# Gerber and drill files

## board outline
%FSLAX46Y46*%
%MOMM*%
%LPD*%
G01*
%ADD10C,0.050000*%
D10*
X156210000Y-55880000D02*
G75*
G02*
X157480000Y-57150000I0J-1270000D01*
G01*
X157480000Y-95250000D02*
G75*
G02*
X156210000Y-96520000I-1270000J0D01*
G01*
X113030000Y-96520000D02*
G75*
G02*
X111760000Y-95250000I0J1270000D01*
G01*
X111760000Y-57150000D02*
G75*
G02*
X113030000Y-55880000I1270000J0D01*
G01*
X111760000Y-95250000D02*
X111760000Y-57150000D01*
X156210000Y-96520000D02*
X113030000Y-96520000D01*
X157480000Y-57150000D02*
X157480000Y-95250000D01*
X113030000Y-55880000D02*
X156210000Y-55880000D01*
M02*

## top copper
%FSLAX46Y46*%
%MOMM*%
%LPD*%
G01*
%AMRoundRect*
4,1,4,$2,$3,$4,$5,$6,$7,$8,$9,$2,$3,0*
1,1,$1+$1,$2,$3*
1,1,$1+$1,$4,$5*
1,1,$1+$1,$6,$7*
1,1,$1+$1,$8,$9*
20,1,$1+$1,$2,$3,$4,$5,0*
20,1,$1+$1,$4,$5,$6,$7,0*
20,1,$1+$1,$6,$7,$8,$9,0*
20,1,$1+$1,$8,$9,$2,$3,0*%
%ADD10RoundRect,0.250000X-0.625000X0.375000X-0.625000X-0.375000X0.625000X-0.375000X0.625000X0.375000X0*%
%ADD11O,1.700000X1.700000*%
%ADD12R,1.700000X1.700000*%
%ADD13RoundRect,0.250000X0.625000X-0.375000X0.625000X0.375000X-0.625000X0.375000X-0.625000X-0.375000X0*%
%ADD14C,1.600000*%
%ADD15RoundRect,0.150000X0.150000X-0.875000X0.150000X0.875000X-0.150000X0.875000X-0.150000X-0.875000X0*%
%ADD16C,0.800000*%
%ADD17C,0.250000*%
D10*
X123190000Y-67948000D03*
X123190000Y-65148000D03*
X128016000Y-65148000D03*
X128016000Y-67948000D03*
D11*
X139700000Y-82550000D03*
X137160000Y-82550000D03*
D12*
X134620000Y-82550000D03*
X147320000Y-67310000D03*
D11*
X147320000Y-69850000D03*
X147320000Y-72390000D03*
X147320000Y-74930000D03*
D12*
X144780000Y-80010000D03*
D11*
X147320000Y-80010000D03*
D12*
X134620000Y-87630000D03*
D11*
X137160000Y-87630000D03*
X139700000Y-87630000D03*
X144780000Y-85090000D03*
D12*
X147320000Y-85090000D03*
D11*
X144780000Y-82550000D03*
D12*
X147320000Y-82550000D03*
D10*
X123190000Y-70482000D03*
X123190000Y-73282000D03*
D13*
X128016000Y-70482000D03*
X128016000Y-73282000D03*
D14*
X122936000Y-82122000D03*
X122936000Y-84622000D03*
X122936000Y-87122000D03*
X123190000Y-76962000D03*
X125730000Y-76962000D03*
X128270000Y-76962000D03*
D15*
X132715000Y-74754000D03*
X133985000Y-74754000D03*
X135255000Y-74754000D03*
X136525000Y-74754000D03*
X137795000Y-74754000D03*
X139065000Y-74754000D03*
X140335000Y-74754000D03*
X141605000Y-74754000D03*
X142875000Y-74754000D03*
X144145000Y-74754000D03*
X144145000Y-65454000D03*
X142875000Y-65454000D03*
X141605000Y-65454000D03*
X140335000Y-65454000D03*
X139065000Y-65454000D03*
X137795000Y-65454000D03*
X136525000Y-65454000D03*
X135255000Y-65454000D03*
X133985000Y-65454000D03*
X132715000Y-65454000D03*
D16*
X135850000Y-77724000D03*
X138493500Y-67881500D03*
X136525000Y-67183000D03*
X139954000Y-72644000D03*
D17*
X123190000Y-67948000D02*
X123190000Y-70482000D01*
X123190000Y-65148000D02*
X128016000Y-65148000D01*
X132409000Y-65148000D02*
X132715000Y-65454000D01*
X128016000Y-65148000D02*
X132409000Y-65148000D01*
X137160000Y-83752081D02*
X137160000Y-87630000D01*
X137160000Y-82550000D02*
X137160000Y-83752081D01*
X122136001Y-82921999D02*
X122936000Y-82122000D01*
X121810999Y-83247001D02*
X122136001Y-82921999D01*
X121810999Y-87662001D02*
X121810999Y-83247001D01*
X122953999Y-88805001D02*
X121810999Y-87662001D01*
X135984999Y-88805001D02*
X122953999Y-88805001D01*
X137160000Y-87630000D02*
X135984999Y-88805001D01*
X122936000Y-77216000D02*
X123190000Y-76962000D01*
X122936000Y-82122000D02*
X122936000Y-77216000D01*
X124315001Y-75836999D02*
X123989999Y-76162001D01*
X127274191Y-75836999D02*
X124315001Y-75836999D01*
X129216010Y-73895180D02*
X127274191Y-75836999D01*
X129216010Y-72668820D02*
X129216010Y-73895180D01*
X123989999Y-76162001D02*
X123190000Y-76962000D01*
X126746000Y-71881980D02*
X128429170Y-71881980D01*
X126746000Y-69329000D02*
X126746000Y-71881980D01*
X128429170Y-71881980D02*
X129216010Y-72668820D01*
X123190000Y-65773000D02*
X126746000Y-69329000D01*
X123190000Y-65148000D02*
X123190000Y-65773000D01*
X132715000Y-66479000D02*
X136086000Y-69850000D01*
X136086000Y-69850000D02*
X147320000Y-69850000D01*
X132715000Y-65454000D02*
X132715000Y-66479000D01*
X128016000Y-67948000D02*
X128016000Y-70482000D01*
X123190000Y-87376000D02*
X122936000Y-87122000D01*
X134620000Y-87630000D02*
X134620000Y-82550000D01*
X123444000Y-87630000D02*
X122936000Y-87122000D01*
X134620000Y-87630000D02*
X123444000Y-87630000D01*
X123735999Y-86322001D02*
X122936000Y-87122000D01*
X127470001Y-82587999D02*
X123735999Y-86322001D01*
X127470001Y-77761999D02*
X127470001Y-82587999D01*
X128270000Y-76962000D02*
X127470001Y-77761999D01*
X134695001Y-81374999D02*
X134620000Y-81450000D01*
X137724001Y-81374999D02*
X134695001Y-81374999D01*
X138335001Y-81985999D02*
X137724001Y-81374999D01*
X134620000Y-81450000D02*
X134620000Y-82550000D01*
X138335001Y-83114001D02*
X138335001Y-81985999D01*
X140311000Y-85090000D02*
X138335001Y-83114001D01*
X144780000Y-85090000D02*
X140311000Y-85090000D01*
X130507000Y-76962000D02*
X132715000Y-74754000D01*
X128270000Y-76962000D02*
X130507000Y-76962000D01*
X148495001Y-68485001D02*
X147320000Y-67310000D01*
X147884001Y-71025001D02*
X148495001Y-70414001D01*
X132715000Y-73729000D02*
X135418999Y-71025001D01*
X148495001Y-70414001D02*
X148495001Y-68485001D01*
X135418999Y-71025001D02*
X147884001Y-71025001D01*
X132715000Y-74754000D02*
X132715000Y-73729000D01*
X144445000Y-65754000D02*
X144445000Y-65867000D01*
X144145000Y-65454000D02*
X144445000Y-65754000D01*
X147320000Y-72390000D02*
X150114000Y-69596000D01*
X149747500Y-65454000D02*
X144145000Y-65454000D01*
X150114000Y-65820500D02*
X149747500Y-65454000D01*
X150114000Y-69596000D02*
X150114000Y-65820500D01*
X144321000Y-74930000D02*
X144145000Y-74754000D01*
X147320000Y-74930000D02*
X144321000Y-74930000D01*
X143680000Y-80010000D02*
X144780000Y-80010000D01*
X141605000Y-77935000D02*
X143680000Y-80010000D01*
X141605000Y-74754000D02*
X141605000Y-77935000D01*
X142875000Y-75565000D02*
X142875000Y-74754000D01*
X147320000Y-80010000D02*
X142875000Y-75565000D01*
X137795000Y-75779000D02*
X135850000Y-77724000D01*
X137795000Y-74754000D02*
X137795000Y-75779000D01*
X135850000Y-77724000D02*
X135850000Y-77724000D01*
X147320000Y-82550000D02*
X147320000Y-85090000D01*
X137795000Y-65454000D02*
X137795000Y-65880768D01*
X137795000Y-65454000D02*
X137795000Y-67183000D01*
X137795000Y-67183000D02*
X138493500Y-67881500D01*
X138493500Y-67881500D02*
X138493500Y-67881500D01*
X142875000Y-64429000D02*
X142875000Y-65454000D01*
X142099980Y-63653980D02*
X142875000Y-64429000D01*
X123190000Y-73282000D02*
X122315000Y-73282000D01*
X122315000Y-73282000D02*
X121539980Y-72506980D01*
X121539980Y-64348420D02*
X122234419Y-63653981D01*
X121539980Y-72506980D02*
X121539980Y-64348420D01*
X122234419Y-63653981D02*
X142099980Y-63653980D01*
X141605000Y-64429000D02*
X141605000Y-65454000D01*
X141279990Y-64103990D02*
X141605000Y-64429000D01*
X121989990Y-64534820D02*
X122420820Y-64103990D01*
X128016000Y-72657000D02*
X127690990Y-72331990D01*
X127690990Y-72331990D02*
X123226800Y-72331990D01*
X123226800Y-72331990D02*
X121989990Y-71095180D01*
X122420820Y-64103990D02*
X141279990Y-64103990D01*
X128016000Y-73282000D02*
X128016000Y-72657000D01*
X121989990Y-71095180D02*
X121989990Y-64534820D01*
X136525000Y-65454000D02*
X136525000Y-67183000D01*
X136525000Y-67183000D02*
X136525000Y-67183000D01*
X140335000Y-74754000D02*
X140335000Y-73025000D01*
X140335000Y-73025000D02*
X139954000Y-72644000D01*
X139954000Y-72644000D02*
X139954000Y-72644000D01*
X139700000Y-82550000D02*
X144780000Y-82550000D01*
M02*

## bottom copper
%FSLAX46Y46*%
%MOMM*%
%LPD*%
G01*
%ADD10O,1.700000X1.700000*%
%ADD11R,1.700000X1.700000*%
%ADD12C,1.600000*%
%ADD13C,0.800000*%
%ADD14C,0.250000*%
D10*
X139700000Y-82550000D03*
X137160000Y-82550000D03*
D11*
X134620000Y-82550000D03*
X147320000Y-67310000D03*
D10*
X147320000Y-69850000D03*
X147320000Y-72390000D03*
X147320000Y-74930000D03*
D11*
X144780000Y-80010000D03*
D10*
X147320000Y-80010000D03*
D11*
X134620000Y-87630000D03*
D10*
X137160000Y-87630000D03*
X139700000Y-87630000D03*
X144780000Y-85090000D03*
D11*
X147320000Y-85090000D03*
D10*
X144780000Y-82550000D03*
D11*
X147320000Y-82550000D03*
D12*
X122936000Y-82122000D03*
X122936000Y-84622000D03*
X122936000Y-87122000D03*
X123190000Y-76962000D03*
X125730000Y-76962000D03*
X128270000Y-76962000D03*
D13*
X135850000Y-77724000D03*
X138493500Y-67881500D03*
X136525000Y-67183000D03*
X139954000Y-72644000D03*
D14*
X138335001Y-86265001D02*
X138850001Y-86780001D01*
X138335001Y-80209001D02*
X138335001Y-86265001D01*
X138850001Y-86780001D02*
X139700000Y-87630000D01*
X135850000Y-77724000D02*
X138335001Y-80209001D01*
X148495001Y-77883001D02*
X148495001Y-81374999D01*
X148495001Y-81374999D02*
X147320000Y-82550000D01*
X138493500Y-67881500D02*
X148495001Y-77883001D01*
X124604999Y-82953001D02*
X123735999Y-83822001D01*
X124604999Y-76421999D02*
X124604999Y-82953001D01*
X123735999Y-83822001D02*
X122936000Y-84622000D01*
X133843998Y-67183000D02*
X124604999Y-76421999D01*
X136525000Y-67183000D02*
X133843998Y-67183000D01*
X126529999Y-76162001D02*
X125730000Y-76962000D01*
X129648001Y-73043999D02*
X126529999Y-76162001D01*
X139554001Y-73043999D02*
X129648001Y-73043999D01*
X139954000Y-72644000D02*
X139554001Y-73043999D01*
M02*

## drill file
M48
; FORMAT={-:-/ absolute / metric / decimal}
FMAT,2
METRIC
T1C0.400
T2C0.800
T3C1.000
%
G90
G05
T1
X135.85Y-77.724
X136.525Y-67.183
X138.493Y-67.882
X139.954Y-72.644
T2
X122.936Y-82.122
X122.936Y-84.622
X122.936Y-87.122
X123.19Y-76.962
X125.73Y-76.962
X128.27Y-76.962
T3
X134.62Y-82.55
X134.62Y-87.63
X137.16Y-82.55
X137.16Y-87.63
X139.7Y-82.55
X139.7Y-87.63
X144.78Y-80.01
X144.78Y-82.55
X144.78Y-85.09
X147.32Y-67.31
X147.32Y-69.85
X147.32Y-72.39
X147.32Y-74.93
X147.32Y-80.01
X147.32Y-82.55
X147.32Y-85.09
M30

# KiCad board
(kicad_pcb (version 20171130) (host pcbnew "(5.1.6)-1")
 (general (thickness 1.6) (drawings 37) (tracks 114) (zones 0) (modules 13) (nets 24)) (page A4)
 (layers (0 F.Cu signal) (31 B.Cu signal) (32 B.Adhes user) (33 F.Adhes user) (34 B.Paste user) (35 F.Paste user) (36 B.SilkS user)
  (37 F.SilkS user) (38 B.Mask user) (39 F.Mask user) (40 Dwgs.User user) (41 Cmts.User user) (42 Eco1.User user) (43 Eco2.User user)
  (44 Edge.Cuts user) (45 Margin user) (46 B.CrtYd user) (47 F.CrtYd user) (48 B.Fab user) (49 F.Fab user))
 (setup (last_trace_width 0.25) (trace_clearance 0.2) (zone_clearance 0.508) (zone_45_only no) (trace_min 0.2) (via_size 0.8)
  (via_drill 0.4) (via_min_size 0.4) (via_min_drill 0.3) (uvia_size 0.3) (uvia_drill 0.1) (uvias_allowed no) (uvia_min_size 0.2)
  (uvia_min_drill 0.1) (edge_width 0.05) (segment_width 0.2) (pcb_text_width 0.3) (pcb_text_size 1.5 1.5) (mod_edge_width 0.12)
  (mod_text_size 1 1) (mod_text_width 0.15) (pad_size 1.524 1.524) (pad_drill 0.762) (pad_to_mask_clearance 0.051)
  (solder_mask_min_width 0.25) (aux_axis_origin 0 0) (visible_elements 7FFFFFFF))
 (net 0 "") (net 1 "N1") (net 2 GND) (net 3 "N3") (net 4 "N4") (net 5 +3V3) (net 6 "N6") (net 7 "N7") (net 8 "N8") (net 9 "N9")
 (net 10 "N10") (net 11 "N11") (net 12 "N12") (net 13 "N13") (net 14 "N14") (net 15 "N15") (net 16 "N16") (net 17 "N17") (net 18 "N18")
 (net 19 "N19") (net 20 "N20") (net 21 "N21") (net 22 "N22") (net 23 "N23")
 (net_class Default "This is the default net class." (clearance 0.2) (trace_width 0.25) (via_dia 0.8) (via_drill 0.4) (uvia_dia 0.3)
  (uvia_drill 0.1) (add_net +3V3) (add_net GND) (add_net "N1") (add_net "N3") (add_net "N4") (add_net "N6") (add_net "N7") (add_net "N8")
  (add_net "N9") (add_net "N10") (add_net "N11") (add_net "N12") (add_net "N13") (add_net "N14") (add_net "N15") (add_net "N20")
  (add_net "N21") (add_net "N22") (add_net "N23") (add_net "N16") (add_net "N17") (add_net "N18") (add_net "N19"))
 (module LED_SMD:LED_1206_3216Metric (layer F.Cu) (at 123.19 66.548 270)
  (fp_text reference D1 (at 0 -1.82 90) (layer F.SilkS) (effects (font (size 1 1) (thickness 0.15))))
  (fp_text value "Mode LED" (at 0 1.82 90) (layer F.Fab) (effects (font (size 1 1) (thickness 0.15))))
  (pad 2 smd roundrect (at 1.4 0 270) (size 1.25 1.75) (layers F.Cu F.Paste F.Mask) (roundrect_rratio 0.2) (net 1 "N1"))
  (pad 1 smd roundrect (at -1.4 0 270) (size 1.25 1.75) (layers F.Cu F.Paste F.Mask) (roundrect_rratio 0.2) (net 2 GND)))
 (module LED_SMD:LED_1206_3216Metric (layer F.Cu) (at 128.016 66.548 270)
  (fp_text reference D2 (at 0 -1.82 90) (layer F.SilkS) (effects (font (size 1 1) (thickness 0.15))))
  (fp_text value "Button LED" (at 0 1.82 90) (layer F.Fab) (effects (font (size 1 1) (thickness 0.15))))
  (pad 1 smd roundrect (at -1.4 0 270) (size 1.25 1.75) (layers F.Cu F.Paste F.Mask) (roundrect_rratio 0.2) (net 2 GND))
  (pad 2 smd roundrect (at 1.4 0 270) (size 1.25 1.75) (layers F.Cu F.Paste F.Mask) (roundrect_rratio 0.2) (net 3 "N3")))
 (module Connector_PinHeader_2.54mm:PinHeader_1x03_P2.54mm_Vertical (layer F.Cu) (at 134.62 82.55 90)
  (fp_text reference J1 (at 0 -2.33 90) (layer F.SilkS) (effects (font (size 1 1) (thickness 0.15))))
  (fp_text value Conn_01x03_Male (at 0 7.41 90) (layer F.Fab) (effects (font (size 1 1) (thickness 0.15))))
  (pad 3 thru_hole oval (at 0 5.08 90) (size 1.7 1.7) (drill 1) (layers *.Cu *.Mask) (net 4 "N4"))
  (pad 2 thru_hole oval (at 0 2.54 90) (size 1.7 1.7) (drill 1) (layers *.Cu *.Mask) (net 2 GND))
  (pad 1 thru_hole rect (at 0 0 90) (size 1.7 1.7) (drill 1) (layers *.Cu *.Mask) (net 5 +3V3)))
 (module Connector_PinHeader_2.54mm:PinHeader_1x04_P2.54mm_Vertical (layer F.Cu) (at 147.32 67.31)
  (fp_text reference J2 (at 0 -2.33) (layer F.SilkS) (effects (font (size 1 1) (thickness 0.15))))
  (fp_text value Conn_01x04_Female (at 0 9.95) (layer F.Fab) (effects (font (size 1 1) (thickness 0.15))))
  (pad 1 thru_hole rect (at 0 0) (size 1.7 1.7) (drill 1) (layers *.Cu *.Mask) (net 5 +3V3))
  (pad 2 thru_hole oval (at 0 2.54) (size 1.7 1.7) (drill 1) (layers *.Cu *.Mask) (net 2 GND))
  (pad 3 thru_hole oval (at 0 5.08) (size 1.7 1.7) (drill 1) (layers *.Cu *.Mask) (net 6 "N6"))
  (pad 4 thru_hole oval (at 0 7.62) (size 1.7 1.7) (drill 1) (layers *.Cu *.Mask) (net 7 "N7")))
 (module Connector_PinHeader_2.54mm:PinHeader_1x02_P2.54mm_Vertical (layer F.Cu) (at 144.78 80.01 90)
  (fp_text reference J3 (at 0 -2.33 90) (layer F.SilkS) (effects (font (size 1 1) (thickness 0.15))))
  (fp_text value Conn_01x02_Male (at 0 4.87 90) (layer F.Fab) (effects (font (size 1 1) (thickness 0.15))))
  (pad 1 thru_hole rect (at 0 0 90) (size 1.7 1.7) (drill 1) (layers *.Cu *.Mask) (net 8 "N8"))
  (pad 2 thru_hole oval (at 0 2.54 90) (size 1.7 1.7) (drill 1) (layers *.Cu *.Mask) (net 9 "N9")))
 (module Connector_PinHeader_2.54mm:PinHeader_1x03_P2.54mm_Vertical (layer F.Cu) (at 134.62 87.63 90)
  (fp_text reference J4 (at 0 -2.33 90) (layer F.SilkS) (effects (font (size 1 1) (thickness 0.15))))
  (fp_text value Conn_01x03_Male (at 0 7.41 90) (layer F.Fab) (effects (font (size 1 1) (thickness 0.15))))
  (pad 1 thru_hole rect (at 0 0 90) (size 1.7 1.7) (drill 1) (layers *.Cu *.Mask) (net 5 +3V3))
  (pad 2 thru_hole oval (at 0 2.54 90) (size 1.7 1.7) (drill 1) (layers *.Cu *.Mask) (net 2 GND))
  (pad 3 thru_hole oval (at 0 5.08 90) (size 1.7 1.7) (drill 1) (layers *.Cu *.Mask) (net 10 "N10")))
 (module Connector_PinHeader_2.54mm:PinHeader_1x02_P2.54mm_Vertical (layer F.Cu) (at 147.32 85.09 270)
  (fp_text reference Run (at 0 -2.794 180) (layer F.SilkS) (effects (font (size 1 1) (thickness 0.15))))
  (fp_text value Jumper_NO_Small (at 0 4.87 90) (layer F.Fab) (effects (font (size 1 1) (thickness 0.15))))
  (pad 2 thru_hole oval (at 0 2.54 270) (size 1.7 1.7) (drill 1) (layers *.Cu *.Mask) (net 5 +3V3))
  (pad 1 thru_hole rect (at 0 0 270) (size 1.7 1.7) (drill 1) (layers *.Cu *.Mask) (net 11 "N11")))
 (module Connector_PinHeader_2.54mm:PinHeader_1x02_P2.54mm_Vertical (layer F.Cu) (at 147.32 82.55 270)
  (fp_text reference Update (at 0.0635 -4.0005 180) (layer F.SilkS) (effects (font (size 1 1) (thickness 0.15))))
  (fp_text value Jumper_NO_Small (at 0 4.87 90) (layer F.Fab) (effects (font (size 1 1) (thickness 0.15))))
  (pad 2 thru_hole oval (at 0 2.54 270) (size 1.7 1.7) (drill 1) (layers *.Cu *.Mask) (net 4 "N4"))
  (pad 1 thru_hole rect (at 0 0 270) (size 1.7 1.7) (drill 1) (layers *.Cu *.Mask) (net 11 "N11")))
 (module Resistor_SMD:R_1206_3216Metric (layer F.Cu) (at 123.19 71.882 270)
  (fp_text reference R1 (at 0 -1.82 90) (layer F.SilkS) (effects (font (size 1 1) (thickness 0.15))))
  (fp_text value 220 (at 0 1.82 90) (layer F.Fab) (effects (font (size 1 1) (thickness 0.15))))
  (pad 1 smd roundrect (at -1.4 0 270) (size 1.25 1.75) (layers F.Cu F.Paste F.Mask) (roundrect_rratio 0.2) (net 1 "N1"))
  (pad 2 smd roundrect (at 1.4 0 270) (size 1.25 1.75) (layers F.Cu F.Paste F.Mask) (roundrect_rratio 0.2) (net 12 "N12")))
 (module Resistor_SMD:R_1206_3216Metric (layer F.Cu) (at 128.016 71.882 90)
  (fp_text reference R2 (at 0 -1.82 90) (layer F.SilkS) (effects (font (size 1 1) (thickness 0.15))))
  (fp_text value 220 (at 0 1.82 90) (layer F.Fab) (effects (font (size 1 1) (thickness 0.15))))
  (pad 2 smd roundrect (at 1.4 0 90) (size 1.25 1.75) (layers F.Cu F.Paste F.Mask) (roundrect_rratio 0.2) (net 3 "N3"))
  (pad 1 smd roundrect (at -1.4 0 90) (size 1.25 1.75) (layers F.Cu F.Paste F.Mask) (roundrect_rratio 0.2) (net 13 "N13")))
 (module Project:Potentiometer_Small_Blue (layer F.Cu) (at 122.936 87.122)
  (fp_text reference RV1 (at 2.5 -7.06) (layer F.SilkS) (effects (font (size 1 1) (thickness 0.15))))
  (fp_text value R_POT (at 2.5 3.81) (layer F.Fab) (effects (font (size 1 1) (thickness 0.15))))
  (pad 3 thru_hole circle (at 0 -5) (size 1.6 1.6) (drill 0.8) (layers *.Cu *.Mask) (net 2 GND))
  (pad 2 thru_hole circle (at 0 -2.5) (size 1.6 1.6) (drill 0.8) (layers *.Cu *.Mask) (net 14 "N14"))
  (pad 1 thru_hole circle (at 0 0) (size 1.6 1.6) (drill 0.8) (layers *.Cu *.Mask) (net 5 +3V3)))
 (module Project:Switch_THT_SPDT (layer F.Cu) (at 125.73 76.962)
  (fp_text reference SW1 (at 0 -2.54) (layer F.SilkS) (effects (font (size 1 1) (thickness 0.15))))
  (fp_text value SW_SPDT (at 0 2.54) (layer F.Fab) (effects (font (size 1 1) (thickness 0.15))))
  (pad 1 thru_hole circle (at -2.54 0) (size 1.6 1.6) (drill 0.8) (layers *.Cu *.Mask) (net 2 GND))
  (pad 2 thru_hole circle (at 0 0) (size 1.6 1.6) (drill 0.8) (layers *.Cu *.Mask) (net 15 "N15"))
  (pad 3 thru_hole circle (at 2.54 0) (size 1.6 1.6) (drill 0.8) (layers *.Cu *.Mask) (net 5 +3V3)))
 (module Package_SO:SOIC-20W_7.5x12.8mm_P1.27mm (layer F.Cu) (at 138.43 70.104 90)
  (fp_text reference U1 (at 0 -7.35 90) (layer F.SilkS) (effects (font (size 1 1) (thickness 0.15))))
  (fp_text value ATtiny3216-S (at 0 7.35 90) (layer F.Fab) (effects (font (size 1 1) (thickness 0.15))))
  (pad 1 smd roundrect (at -4.65 -5.715 90) (size 2.05 0.6) (layers F.Cu F.Paste F.Mask) (roundrect_rratio 0.25) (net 5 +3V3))
  (pad 2 smd roundrect (at -4.65 -4.445 90) (size 2.05 0.6) (layers F.Cu F.Paste F.Mask) (roundrect_rratio 0.25) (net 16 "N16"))
  (pad 3 smd roundrect (at -4.65 -3.175 90) (size 2.05 0.6) (layers F.Cu F.Paste F.Mask) (roundrect_rratio 0.25) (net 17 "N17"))
  (pad 4 smd roundrect (at -4.65 -1.905 90) (size 2.05 0.6) (layers F.Cu F.Paste F.Mask) (roundrect_rratio 0.25) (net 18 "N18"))
  (pad 5 smd roundrect (at -4.65 -0.635 90) (size 2.05 0.6) (layers F.Cu F.Paste F.Mask) (roundrect_rratio 0.25) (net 10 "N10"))
  (pad 6 smd roundrect (at -4.65 0.635 90) (size 2.05 0.6) (layers F.Cu F.Paste F.Mask) (roundrect_rratio 0.25) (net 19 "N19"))
  (pad 7 smd roundrect (at -4.65 1.905 90) (size 2.05 0.6) (layers F.Cu F.Paste F.Mask) (roundrect_rratio 0.25) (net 15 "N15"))
  (pad 8 smd roundrect (at -4.65 3.175 90) (size 2.05 0.6) (layers F.Cu F.Paste F.Mask) (roundrect_rratio 0.25) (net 8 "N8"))
  (pad 9 smd roundrect (at -4.65 4.445 90) (size 2.05 0.6) (layers F.Cu F.Paste F.Mask) (roundrect_rratio 0.25) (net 9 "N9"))
  (pad 10 smd roundrect (at -4.65 5.715 90) (size 2.05 0.6) (layers F.Cu F.Paste F.Mask) (roundrect_rratio 0.25) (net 7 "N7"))
  (pad 11 smd roundrect (at 4.65 5.715 90) (size 2.05 0.6) (layers F.Cu F.Paste F.Mask) (roundrect_rratio 0.25) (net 6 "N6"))
  (pad 12 smd roundrect (at 4.65 4.445 90) (size 2.05 0.6) (layers F.Cu F.Paste F.Mask) (roundrect_rratio 0.25) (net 12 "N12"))
  (pad 13 smd roundrect (at 4.65 3.175 90) (size 2.05 0.6) (layers F.Cu F.Paste F.Mask) (roundrect_rratio 0.25) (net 13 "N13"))
  (pad 14 smd roundrect (at 4.65 1.905 90) (size 2.05 0.6) (layers F.Cu F.Paste F.Mask) (roundrect_rratio 0.25) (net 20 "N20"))
  (pad 15 smd roundrect (at 4.65 0.635 90) (size 2.05 0.6) (layers F.Cu F.Paste F.Mask) (roundrect_rratio 0.25) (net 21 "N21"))
  (pad 16 smd roundrect (at 4.65 -0.635 90) (size 2.05 0.6) (layers F.Cu F.Paste F.Mask) (roundrect_rratio 0.25) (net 11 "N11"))
  (pad 17 smd roundrect (at 4.65 -1.905 90) (size 2.05 0.6) (layers F.Cu F.Paste F.Mask) (roundrect_rratio 0.25) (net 14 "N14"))
  (pad 18 smd roundrect (at 4.65 -3.175 90) (size 2.05 0.6) (layers F.Cu F.Paste F.Mask) (roundrect_rratio 0.25) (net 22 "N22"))
  (pad 19 smd roundrect (at 4.65 -4.445 90) (size 2.05 0.6) (layers F.Cu F.Paste F.Mask) (roundrect_rratio 0.25) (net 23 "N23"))
  (pad 20 smd roundrect (at 4.65 -5.715 90) (size 2.05 0.6) (layers F.Cu F.Paste F.Mask) (roundrect_rratio 0.25) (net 2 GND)))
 (gr_arc (start 156.21 57.15) (end 157.48 57.15) (angle -90) (layer Edge.Cuts) (width 0.05))
 (gr_arc (start 156.21 95.25) (end 156.21 96.52) (angle -90) (layer Edge.Cuts) (width 0.05))
 (gr_arc (start 113.03 95.25) (end 111.76 95.25) (angle -90) (layer Edge.Cuts) (width 0.05))
 (gr_arc (start 113.03 57.15) (end 113.03 55.88) (angle -90) (layer Edge.Cuts) (width 0.05))
 (gr_line (start 111.76 95.25) (end 111.76 57.15) (layer Edge.Cuts) (width 0.05))
 (gr_line (start 156.21 96.52) (end 113.03 96.52) (layer Edge.Cuts) (width 0.05))
 (gr_line (start 157.48 57.15) (end 157.48 95.25) (layer Edge.Cuts) (width 0.05))
 (gr_line (start 113.03 55.88) (end 156.21 55.88) (layer Edge.Cuts) (width 0.05))
 (segment (start 123.19 67.948) (end 123.19 70.482) (width 0.25) (layer F.Cu) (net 1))
 (segment (start 123.19 65.148) (end 128.016 65.148) (width 0.25) (layer F.Cu) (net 2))
 (segment (start 132.409 65.148) (end 132.715 65.454) (width 0.25) (layer F.Cu) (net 2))
 (segment (start 128.016 65.148) (end 132.409 65.148) (width 0.25) (layer F.Cu) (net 2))
 (segment (start 137.16 83.752081) (end 137.16 87.63) (width 0.25) (layer F.Cu) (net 2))
 (segment (start 137.16 82.55) (end 137.16 83.752081) (width 0.25) (layer F.Cu) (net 2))
 (segment (start 122.136001 82.921999) (end 122.936 82.122) (width 0.25) (layer F.Cu) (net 2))
 (segment (start 121.810999 83.247001) (end 122.136001 82.921999) (width 0.25) (layer F.Cu) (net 2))
 (segment (start 121.810999 87.662001) (end 121.810999 83.247001) (width 0.25) (layer F.Cu) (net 2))
 (segment (start 122.953999 88.805001) (end 121.810999 87.662001) (width 0.25) (layer F.Cu) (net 2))
 (segment (start 135.984999 88.805001) (end 122.953999 88.805001) (width 0.25) (layer F.Cu) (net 2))
 (segment (start 137.16 87.63) (end 135.984999 88.805001) (width 0.25) (layer F.Cu) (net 2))
 (segment (start 122.936 77.216) (end 123.19 76.962) (width 0.25) (layer F.Cu) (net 2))
 (segment (start 122.936 82.122) (end 122.936 77.216) (width 0.25) (layer F.Cu) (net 2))
 (segment (start 124.315001 75.836999) (end 123.989999 76.162001) (width 0.25) (layer F.Cu) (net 2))
 (segment (start 127.274191 75.836999) (end 124.315001 75.836999) (width 0.25) (layer F.Cu) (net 2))
 (segment (start 129.21601 73.89518) (end 127.274191 75.836999) (width 0.25) (layer F.Cu) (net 2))
 (segment (start 129.21601 72.66882) (end 129.21601 73.89518) (width 0.25) (layer F.Cu) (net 2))
 (segment (start 123.989999 76.162001) (end 123.19 76.962) (width 0.25) (layer F.Cu) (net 2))
 (segment (start 126.746 71.88198) (end 128.42917 71.88198) (width 0.25) (layer F.Cu) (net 2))
 (segment (start 126.746 69.329) (end 126.746 71.88198) (width 0.25) (layer F.Cu) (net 2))
 (segment (start 128.42917 71.88198) (end 129.21601 72.66882) (width 0.25) (layer F.Cu) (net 2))
 (segment (start 123.19 65.773) (end 126.746 69.329) (width 0.25) (layer F.Cu) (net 2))
 (segment (start 123.19 65.148) (end 123.19 65.773) (width 0.25) (layer F.Cu) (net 2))
 (segment (start 132.715 66.479) (end 136.086 69.85) (width 0.25) (layer F.Cu) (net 2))
 (segment (start 136.086 69.85) (end 147.32 69.85) (width 0.25) (layer F.Cu) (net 2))
 (segment (start 132.715 65.454) (end 132.715 66.479) (width 0.25) (layer F.Cu) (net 2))
 (segment (start 128.016 67.948) (end 128.016 70.482) (width 0.25) (layer F.Cu) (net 3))
 (segment (start 123.19 87.376) (end 122.936 87.122) (width 0.25) (layer F.Cu) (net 5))
 (segment (start 134.62 87.63) (end 134.62 82.55) (width 0.25) (layer F.Cu) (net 5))
 (segment (start 123.444 87.63) (end 122.936 87.122) (width 0.25) (layer F.Cu) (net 5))
 (segment (start 134.62 87.63) (end 123.444 87.63) (width 0.25) (layer F.Cu) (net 5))
 (segment (start 123.735999 86.322001) (end 122.936 87.122) (width 0.25) (layer F.Cu) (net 5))
 (segment (start 127.470001 82.587999) (end 123.735999 86.322001) (width 0.25) (layer F.Cu) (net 5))
 (segment (start 127.470001 77.761999) (end 127.470001 82.587999) (width 0.25) (layer F.Cu) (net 5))
 (segment (start 128.27 76.962) (end 127.470001 77.761999) (width 0.25) (layer F.Cu) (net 5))
 (segment (start 134.695001 81.374999) (end 134.62 81.45) (width 0.25) (layer F.Cu) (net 5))
 (segment (start 137.724001 81.374999) (end 134.695001 81.374999) (width 0.25) (layer F.Cu) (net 5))
 (segment (start 138.335001 81.985999) (end 137.724001 81.374999) (width 0.25) (layer F.Cu) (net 5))
 (segment (start 134.62 81.45) (end 134.62 82.55) (width 0.25) (layer F.Cu) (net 5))
 (segment (start 138.335001 83.114001) (end 138.335001 81.985999) (width 0.25) (layer F.Cu) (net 5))
 (segment (start 140.311 85.09) (end 138.335001 83.114001) (width 0.25) (layer F.Cu) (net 5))
 (segment (start 144.78 85.09) (end 140.311 85.09) (width 0.25) (layer F.Cu) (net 5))
 (segment (start 130.507 76.962) (end 132.715 74.754) (width 0.25) (layer F.Cu) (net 5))
 (segment (start 128.27 76.962) (end 130.507 76.962) (width 0.25) (layer F.Cu) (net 5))
 (segment (start 148.495001 68.485001) (end 147.32 67.31) (width 0.25) (layer F.Cu) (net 5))
 (segment (start 147.884001 71.025001) (end 148.495001 70.414001) (width 0.25) (layer F.Cu) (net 5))
 (segment (start 132.715 73.729) (end 135.418999 71.025001) (width 0.25) (layer F.Cu) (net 5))
 (segment (start 148.495001 70.414001) (end 148.495001 68.485001) (width 0.25) (layer F.Cu) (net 5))
 (segment (start 135.418999 71.025001) (end 147.884001 71.025001) (width 0.25) (layer F.Cu) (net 5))
 (segment (start 132.715 74.754) (end 132.715 73.729) (width 0.25) (layer F.Cu) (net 5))
 (segment (start 144.445 65.754) (end 144.445 65.867) (width 0.25) (layer F.Cu) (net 6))
 (segment (start 144.145 65.454) (end 144.445 65.754) (width 0.25) (layer F.Cu) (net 6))
 (segment (start 147.32 72.39) (end 150.114 69.596) (width 0.25) (layer F.Cu) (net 6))
 (segment (start 149.7475 65.454) (end 144.145 65.454) (width 0.25) (layer F.Cu) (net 6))
 (segment (start 150.114 65.8205) (end 149.7475 65.454) (width 0.25) (layer F.Cu) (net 6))
 (segment (start 150.114 69.596) (end 150.114 65.8205) (width 0.25) (layer F.Cu) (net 6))
 (segment (start 144.321 74.93) (end 144.145 74.754) (width 0.25) (layer F.Cu) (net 7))
 (segment (start 147.32 74.93) (end 144.321 74.93) (width 0.25) (layer F.Cu) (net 7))
 (segment (start 143.68 80.01) (end 144.78 80.01) (width 0.25) (layer F.Cu) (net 8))
 (segment (start 141.605 77.935) (end 143.68 80.01) (width 0.25) (layer F.Cu) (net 8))
 (segment (start 141.605 74.754) (end 141.605 77.935) (width 0.25) (layer F.Cu) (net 8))
 (segment (start 142.875 75.565) (end 142.875 74.754) (width 0.25) (layer F.Cu) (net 9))
 (segment (start 147.32 80.01) (end 142.875 75.565) (width 0.25) (layer F.Cu) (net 9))
 (segment (start 137.795 75.779) (end 135.85 77.724) (width 0.25) (layer F.Cu) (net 10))
 (segment (start 137.795 74.754) (end 137.795 75.779) (width 0.25) (layer F.Cu) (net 10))
 (segment (start 135.85 77.724) (end 135.85 77.724) (width 0.25) (layer F.Cu) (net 10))
 (via (at 135.85 77.724) (size 0.8) (drill 0.4) (layers F.Cu B.Cu) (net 10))
 (segment (start 138.335001 86.265001) (end 138.850001 86.780001) (width 0.25) (layer B.Cu) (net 10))
 (segment (start 138.335001 80.209001) (end 138.335001 86.265001) (width 0.25) (layer B.Cu) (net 10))
 (segment (start 138.850001 86.780001) (end 139.7 87.63) (width 0.25) (layer B.Cu) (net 10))
 (segment (start 135.85 77.724) (end 138.335001 80.209001) (width 0.25) (layer B.Cu) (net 10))
 (segment (start 147.32 82.55) (end 147.32 85.09) (width 0.25) (layer F.Cu) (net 11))
 (segment (start 137.795 65.454) (end 137.795 65.880768) (width 0.25) (layer F.Cu) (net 11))
 (segment (start 137.795 65.454) (end 137.795 67.183) (width 0.25) (layer F.Cu) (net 11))
 (segment (start 137.795 67.183) (end 138.4935 67.8815) (width 0.25) (layer F.Cu) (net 11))
 (segment (start 138.4935 67.8815) (end 138.4935 67.8815) (width 0.25) (layer F.Cu) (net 11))
 (via (at 138.4935 67.8815) (size 0.8) (drill 0.4) (layers F.Cu B.Cu) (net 11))
 (segment (start 148.495001 77.883001) (end 148.495001 81.374999) (width 0.25) (layer B.Cu) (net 11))
 (segment (start 148.495001 81.374999) (end 147.32 82.55) (width 0.25) (layer B.Cu) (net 11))
 (segment (start 138.4935 67.8815) (end 148.495001 77.883001) (width 0.25) (layer B.Cu) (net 11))
 (segment (start 142.875 64.429) (end 142.875 65.454) (width 0.25) (layer F.Cu) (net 12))
 (segment (start 142.09998 63.65398) (end 142.875 64.429) (width 0.25) (layer F.Cu) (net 12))
 (segment (start 123.19 73.282) (end 122.315 73.282) (width 0.25) (layer F.Cu) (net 12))
 (segment (start 122.315 73.282) (end 121.53998 72.50698) (width 0.25) (layer F.Cu) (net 12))
 (segment (start 121.53998 64.34842) (end 122.234419 63.653981) (width 0.25) (layer F.Cu) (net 12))
 (segment (start 121.53998 72.50698) (end 121.53998 64.34842) (width 0.25) (layer F.Cu) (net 12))
 (segment (start 122.234419 63.653981) (end 142.09998 63.65398) (width 0.25) (layer F.Cu) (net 12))
 (segment (start 141.605 64.429) (end 141.605 65.454) (width 0.25) (layer F.Cu) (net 13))
 (segment (start 141.27999 64.10399) (end 141.605 64.429) (width 0.25) (layer F.Cu) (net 13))
 (segment (start 121.98999 64.53482) (end 122.42082 64.10399) (width 0.25) (layer F.Cu) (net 13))
 (segment (start 128.016 72.657) (end 127.69099 72.33199) (width 0.25) (layer F.Cu) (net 13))
 (segment (start 127.69099 72.33199) (end 123.2268 72.33199) (width 0.25) (layer F.Cu) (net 13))
 (segment (start 123.2268 72.33199) (end 121.98999 71.09518) (width 0.25) (layer F.Cu) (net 13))
 (segment (start 122.42082 64.10399) (end 141.27999 64.10399) (width 0.25) (layer F.Cu) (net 13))
 (segment (start 128.016 73.282) (end 128.016 72.657) (width 0.25) (layer F.Cu) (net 13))
 (segment (start 121.98999 71.09518) (end 121.98999 64.53482) (width 0.25) (layer F.Cu) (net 13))
 (segment (start 136.525 65.454) (end 136.525 67.183) (width 0.25) (layer F.Cu) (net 14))
 (segment (start 136.525 67.183) (end 136.525 67.183) (width 0.25) (layer F.Cu) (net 14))
 (via (at 136.525 67.183) (size 0.8) (drill 0.4) (layers F.Cu B.Cu) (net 14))
 (segment (start 124.604999 82.953001) (end 123.735999 83.822001) (width 0.25) (layer B.Cu) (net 14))
 (segment (start 124.604999 76.421999) (end 124.604999 82.953001) (width 0.25) (layer B.Cu) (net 14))
 (segment (start 123.735999 83.822001) (end 122.936 84.622) (width 0.25) (layer B.Cu) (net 14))
 (segment (start 133.843998 67.183) (end 124.604999 76.421999) (width 0.25) (layer B.Cu) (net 14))
 (segment (start 136.525 67.183) (end 133.843998 67.183) (width 0.25) (layer B.Cu) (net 14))
 (segment (start 140.335 74.754) (end 140.335 73.025) (width 0.25) (layer F.Cu) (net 15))
 (segment (start 140.335 73.025) (end 139.954 72.644) (width 0.25) (layer F.Cu) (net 15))
 (segment (start 139.954 72.644) (end 139.954 72.644) (width 0.25) (layer F.Cu) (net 15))
 (via (at 139.954 72.644) (size 0.8) (drill 0.4) (layers F.Cu B.Cu) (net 15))
 (segment (start 126.529999 76.162001) (end 125.73 76.962) (width 0.25) (layer B.Cu) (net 15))
 (segment (start 129.648001 73.043999) (end 126.529999 76.162001) (width 0.25) (layer B.Cu) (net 15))
 (segment (start 139.554001 73.043999) (end 129.648001 73.043999) (width 0.25) (layer B.Cu) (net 15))
 (segment (start 139.954 72.644) (end 139.554001 73.043999) (width 0.25) (layer B.Cu) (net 15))
 (segment (start 139.7 82.55) (end 144.78 82.55) (width 0.25) (layer F.Cu) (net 4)))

